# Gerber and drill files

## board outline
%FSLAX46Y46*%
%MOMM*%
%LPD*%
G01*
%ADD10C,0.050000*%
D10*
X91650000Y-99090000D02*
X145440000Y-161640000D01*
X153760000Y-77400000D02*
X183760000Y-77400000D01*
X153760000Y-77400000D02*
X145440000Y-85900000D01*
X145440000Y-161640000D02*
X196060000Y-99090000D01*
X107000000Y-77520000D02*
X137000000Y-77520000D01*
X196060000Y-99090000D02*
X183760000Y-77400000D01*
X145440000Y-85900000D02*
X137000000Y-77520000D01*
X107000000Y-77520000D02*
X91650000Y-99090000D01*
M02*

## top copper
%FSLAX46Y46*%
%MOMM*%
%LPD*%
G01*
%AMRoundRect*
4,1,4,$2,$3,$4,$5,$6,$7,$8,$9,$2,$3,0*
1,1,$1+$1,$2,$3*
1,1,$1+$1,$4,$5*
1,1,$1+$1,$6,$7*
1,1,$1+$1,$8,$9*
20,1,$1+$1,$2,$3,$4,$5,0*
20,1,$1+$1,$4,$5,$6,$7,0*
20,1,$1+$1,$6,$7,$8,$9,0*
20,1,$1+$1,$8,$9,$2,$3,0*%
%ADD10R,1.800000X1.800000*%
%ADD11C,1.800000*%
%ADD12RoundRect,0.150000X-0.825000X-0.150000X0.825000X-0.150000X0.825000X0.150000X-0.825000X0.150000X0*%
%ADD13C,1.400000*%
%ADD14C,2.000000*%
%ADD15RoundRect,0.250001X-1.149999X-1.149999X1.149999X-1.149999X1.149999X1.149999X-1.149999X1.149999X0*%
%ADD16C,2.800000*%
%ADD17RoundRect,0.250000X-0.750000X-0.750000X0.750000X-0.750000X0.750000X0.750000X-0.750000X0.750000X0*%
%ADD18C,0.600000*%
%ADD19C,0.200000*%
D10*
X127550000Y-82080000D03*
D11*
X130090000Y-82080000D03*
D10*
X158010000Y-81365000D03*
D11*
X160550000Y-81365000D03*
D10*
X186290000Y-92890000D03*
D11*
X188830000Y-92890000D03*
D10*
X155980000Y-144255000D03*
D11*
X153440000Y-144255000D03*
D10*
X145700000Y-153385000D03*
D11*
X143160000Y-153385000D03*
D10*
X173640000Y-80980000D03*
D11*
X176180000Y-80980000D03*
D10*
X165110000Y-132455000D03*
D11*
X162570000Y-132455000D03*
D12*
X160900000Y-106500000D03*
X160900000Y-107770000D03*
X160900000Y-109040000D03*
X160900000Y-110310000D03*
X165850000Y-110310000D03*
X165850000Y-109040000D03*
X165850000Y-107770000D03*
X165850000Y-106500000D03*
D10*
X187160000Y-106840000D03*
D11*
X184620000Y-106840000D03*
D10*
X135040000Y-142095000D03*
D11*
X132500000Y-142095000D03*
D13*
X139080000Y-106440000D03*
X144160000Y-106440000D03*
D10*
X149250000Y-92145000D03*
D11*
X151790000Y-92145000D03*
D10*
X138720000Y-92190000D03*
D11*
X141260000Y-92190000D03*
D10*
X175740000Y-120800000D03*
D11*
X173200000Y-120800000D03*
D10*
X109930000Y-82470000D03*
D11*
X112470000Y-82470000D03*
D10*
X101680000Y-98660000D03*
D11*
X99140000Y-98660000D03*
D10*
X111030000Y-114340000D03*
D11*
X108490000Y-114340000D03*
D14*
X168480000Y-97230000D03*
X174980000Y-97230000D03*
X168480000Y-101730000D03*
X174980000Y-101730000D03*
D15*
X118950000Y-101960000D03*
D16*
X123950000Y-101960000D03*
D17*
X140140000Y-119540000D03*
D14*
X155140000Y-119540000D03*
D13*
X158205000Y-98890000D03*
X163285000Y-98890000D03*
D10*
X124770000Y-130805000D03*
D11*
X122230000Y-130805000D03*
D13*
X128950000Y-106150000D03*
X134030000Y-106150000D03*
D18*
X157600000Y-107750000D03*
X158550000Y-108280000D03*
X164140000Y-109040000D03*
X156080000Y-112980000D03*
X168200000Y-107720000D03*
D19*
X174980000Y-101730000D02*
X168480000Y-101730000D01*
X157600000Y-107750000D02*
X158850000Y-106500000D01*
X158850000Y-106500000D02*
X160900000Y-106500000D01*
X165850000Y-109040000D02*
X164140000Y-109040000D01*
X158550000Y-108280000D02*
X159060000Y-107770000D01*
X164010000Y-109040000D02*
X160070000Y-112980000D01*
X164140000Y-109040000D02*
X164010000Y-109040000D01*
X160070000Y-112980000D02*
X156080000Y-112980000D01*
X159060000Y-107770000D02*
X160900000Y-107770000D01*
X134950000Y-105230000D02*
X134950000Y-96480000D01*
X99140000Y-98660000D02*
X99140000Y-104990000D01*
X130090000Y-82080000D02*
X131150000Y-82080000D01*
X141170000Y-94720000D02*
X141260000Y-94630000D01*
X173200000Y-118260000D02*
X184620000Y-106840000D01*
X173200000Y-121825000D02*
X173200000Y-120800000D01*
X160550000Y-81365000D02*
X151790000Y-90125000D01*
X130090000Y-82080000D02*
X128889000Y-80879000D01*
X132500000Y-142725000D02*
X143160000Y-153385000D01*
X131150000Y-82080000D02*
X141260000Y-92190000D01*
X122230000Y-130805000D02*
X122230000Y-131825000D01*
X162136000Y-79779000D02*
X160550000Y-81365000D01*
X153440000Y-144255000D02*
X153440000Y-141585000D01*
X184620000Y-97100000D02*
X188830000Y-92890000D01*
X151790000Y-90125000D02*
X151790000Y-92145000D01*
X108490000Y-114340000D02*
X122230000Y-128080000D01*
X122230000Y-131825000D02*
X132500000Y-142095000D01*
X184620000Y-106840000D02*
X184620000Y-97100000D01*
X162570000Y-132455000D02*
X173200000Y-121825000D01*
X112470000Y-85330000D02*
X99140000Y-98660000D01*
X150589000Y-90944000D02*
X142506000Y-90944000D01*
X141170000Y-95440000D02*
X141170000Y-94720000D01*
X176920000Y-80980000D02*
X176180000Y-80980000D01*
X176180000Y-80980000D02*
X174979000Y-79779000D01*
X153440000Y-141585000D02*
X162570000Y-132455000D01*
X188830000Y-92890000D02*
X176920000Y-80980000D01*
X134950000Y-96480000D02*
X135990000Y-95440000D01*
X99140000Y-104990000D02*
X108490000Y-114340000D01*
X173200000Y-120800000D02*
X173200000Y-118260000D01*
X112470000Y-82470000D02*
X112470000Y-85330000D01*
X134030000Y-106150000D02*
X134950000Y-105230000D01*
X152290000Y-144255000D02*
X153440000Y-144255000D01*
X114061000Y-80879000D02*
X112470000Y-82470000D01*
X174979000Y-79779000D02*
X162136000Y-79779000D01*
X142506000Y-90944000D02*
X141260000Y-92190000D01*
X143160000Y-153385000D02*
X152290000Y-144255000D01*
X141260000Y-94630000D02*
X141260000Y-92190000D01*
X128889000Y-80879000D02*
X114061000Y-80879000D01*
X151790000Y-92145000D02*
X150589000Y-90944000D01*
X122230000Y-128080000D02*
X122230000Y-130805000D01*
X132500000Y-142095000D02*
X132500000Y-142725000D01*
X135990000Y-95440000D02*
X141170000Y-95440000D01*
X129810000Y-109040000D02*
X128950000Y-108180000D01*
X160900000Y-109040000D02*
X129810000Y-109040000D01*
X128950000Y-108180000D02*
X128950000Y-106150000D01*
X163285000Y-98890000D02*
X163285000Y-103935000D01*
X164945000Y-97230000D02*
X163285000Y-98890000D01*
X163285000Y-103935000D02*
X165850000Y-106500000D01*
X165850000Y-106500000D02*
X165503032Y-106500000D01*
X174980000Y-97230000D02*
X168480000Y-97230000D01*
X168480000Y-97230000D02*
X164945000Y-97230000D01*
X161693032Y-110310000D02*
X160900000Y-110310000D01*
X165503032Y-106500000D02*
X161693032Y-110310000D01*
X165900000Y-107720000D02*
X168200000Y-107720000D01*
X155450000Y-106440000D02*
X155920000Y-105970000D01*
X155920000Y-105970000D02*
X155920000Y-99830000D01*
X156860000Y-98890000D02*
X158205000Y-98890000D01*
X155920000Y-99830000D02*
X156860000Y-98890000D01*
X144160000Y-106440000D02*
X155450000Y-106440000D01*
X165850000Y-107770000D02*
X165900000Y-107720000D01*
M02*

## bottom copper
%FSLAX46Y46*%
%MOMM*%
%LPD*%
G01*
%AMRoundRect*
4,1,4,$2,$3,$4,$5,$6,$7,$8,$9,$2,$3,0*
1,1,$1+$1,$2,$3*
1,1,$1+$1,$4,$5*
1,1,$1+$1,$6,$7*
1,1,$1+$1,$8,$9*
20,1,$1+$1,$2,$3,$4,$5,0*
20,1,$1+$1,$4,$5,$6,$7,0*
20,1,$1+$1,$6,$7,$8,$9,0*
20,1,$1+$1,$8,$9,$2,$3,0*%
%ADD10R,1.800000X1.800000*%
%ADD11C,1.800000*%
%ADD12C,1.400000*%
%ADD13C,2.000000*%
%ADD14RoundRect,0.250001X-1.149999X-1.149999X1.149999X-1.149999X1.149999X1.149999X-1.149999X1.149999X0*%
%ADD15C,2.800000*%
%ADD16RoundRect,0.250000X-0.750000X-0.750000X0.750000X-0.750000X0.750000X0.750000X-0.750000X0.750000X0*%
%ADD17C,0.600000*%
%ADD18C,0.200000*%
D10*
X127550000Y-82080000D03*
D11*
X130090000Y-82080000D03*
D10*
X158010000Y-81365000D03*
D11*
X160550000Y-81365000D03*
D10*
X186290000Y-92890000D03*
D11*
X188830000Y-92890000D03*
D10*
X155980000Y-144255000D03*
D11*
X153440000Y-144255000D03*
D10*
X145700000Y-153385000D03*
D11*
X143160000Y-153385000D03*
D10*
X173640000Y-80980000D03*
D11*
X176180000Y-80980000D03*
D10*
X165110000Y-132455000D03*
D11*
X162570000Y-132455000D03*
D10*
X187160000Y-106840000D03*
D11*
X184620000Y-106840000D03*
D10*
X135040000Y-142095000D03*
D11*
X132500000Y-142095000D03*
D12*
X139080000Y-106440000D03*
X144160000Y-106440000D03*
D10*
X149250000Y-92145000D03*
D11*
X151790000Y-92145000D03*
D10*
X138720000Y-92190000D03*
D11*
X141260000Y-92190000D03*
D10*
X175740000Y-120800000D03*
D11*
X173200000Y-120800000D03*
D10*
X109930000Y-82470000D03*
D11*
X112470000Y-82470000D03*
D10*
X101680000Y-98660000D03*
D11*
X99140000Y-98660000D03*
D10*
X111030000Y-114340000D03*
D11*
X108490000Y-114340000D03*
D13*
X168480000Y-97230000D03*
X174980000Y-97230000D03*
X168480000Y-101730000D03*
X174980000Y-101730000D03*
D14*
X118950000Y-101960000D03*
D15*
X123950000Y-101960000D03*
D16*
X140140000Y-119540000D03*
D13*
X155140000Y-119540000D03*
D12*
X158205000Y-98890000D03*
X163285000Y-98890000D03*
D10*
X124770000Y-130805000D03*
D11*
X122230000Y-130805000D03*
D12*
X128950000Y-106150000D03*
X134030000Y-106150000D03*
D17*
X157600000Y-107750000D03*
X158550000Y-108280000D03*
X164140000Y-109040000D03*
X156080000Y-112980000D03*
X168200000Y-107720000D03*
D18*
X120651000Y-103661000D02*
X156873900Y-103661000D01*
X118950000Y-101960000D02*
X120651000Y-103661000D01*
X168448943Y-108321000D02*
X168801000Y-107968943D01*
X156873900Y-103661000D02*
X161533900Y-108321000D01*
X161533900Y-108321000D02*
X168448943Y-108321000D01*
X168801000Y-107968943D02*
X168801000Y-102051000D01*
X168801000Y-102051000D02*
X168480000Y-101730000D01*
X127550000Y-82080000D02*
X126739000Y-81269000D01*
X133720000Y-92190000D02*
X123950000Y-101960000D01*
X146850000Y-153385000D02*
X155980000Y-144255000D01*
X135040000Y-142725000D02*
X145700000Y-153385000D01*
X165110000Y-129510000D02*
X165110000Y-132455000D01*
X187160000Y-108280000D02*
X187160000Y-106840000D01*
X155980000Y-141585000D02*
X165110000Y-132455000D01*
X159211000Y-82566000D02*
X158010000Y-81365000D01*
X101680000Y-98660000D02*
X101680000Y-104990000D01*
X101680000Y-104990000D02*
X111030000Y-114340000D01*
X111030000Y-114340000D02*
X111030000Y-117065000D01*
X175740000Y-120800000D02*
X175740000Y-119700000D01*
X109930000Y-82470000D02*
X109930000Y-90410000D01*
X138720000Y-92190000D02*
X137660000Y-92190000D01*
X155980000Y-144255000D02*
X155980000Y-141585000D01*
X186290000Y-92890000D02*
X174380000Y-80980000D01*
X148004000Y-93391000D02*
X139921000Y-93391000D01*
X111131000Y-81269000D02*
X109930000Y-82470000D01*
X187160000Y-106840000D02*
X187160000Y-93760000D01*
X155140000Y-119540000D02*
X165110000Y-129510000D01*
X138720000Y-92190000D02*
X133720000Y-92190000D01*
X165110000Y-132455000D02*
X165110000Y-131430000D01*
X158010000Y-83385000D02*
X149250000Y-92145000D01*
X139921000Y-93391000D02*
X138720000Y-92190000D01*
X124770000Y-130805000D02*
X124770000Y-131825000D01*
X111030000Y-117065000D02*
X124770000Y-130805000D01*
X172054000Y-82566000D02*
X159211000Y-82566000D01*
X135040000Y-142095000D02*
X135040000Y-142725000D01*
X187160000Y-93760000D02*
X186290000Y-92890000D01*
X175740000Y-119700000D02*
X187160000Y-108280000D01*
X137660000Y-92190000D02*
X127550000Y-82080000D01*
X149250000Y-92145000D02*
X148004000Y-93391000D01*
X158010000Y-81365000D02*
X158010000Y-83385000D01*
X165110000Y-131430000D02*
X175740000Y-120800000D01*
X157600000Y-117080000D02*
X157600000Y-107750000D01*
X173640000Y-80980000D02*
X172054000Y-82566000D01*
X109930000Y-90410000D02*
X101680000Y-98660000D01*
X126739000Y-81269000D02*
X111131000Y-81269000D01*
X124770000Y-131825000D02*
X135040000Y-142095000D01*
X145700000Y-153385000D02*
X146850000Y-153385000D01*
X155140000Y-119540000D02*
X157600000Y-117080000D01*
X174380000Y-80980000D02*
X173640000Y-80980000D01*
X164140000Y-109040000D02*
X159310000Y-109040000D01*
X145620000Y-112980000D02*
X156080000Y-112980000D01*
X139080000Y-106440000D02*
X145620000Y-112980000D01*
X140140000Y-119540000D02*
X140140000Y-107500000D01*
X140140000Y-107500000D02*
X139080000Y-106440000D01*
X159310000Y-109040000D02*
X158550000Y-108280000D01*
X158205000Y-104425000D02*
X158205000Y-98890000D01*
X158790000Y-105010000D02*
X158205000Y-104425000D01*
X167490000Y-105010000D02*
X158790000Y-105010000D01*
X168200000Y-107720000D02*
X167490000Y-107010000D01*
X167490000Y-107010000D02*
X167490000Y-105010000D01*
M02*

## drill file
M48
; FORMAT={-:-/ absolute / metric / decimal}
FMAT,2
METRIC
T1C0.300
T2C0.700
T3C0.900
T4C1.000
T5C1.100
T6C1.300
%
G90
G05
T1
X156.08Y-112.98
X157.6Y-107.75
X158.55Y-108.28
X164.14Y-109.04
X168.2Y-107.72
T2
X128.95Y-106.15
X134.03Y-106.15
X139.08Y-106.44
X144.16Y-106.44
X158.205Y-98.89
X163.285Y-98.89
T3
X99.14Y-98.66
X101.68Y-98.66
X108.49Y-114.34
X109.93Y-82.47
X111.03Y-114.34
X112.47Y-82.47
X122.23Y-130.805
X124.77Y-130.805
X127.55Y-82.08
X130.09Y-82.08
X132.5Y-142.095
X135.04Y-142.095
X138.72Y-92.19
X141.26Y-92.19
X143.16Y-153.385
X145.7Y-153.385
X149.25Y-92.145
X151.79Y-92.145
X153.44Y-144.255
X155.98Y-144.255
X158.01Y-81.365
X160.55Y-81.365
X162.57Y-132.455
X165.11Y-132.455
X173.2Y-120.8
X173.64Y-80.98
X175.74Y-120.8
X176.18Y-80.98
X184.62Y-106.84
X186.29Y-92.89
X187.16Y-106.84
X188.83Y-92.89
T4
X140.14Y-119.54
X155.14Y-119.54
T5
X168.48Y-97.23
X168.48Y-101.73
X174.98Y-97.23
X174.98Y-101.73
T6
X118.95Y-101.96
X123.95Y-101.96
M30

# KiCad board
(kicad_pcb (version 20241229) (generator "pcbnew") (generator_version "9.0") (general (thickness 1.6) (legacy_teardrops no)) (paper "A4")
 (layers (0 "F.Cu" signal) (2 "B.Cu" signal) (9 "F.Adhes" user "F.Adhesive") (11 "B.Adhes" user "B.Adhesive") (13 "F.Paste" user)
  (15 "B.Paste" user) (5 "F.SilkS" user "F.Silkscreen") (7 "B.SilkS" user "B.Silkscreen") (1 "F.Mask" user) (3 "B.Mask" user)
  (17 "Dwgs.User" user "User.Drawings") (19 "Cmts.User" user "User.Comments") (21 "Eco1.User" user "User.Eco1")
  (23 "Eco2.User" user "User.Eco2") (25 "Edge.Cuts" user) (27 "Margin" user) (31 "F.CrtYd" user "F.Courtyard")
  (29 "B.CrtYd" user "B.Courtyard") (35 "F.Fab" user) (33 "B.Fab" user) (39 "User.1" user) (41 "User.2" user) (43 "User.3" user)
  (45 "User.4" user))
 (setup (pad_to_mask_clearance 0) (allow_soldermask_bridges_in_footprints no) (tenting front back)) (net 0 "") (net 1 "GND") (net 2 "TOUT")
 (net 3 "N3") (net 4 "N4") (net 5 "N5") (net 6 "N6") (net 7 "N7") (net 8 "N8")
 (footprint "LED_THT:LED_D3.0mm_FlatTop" (layer "F.Cu") (at 127.55 82.08)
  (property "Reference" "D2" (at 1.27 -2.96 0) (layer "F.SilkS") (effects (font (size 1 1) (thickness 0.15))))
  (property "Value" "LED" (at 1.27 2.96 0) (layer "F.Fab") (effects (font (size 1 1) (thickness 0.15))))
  (pad "1" thru_hole rect (at 0 0) (size 1.8 1.8) (drill 0.9) (layers "*.Cu" "*.Mask") (remove_unused_layers no) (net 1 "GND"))
  (pad "2" thru_hole circle (at 2.54 0) (size 1.8 1.8) (drill 0.9) (layers "*.Cu" "*.Mask") (remove_unused_layers no) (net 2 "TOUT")))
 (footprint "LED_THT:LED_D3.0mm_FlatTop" (layer "F.Cu") (at 158.01 81.365)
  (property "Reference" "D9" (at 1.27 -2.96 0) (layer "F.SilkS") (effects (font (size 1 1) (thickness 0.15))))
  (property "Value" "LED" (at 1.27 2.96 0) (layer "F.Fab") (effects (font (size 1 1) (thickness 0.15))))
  (pad "1" thru_hole rect (at 0 0) (size 1.8 1.8) (drill 0.9) (layers "*.Cu" "*.Mask") (remove_unused_layers no) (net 1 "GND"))
  (pad "2" thru_hole circle (at 2.54 0) (size 1.8 1.8) (drill 0.9) (layers "*.Cu" "*.Mask") (remove_unused_layers no) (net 2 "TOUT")))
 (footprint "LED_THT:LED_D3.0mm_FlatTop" (layer "F.Cu") (at 186.29 92.89)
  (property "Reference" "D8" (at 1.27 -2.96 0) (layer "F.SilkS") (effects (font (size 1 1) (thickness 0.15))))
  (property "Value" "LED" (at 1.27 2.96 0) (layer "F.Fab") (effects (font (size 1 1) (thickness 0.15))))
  (pad "1" thru_hole rect (at 0 0) (size 1.8 1.8) (drill 0.9) (layers "*.Cu" "*.Mask") (remove_unused_layers no) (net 1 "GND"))
  (pad "2" thru_hole circle (at 2.54 0) (size 1.8 1.8) (drill 0.9) (layers "*.Cu" "*.Mask") (remove_unused_layers no) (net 2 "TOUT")))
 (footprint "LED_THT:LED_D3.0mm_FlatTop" (layer "F.Cu") (at 155.98 144.255 180)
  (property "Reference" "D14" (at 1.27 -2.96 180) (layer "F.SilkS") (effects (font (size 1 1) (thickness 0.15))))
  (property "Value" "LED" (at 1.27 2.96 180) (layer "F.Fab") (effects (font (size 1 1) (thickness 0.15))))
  (pad "1" thru_hole rect (at 0 0 180) (size 1.8 1.8) (drill 0.9) (layers "*.Cu" "*.Mask") (remove_unused_layers no) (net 1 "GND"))
  (pad "2" thru_hole circle (at 2.54 0 180) (size 1.8 1.8) (drill 0.9) (layers "*.Cu" "*.Mask") (remove_unused_layers no) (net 2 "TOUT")))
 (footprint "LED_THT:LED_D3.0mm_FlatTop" (layer "F.Cu") (at 145.7 153.385 180)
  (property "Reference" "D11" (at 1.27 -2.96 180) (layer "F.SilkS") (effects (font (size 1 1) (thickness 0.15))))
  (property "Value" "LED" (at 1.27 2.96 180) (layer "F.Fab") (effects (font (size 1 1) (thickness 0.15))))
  (pad "1" thru_hole rect (at 0 0 180) (size 1.8 1.8) (drill 0.9) (layers "*.Cu" "*.Mask") (remove_unused_layers no) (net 1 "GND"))
  (pad "2" thru_hole circle (at 2.54 0 180) (size 1.8 1.8) (drill 0.9) (layers "*.Cu" "*.Mask") (remove_unused_layers no) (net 2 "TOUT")))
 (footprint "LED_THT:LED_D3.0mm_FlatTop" (layer "F.Cu") (at 173.64 80.98)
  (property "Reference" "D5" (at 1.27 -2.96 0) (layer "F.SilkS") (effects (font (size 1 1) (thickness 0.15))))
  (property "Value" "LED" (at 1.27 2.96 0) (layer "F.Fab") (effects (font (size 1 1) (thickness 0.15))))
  (pad "1" thru_hole rect (at 0 0) (size 1.8 1.8) (drill 0.9) (layers "*.Cu" "*.Mask") (remove_unused_layers no) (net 1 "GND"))
  (pad "2" thru_hole circle (at 2.54 0) (size 1.8 1.8) (drill 0.9) (layers "*.Cu" "*.Mask") (remove_unused_layers no) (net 2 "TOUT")))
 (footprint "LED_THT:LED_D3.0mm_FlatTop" (layer "F.Cu") (at 165.11 132.455 180)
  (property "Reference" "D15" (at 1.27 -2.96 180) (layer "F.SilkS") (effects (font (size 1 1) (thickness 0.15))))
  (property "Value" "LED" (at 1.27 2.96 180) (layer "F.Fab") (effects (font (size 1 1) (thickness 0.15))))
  (pad "1" thru_hole rect (at 0 0 180) (size 1.8 1.8) (drill 0.9) (layers "*.Cu" "*.Mask") (remove_unused_layers no) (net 1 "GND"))
  (pad "2" thru_hole circle (at 2.54 0 180) (size 1.8 1.8) (drill 0.9) (layers "*.Cu" "*.Mask") (remove_unused_layers no) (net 2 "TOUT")))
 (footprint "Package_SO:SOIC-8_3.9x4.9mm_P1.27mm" (layer "F.Cu") (at 163.375 108.405)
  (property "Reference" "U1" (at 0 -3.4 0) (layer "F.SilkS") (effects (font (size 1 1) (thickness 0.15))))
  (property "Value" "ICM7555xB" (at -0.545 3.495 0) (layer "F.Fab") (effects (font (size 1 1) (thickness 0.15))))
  (pad "1" smd roundrect (at -2.475 -1.905) (size 1.95 0.6) (layers "F.Cu" "F.Mask" "F.Paste") (roundrect_rratio 0.25) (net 1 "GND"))
  (pad "2" smd roundrect (at -2.475 -0.635) (size 1.95 0.6) (layers "F.Cu" "F.Mask" "F.Paste") (roundrect_rratio 0.25) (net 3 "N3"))
  (pad "3" smd roundrect (at -2.475 0.635) (size 1.95 0.6) (layers "F.Cu" "F.Mask" "F.Paste") (roundrect_rratio 0.25) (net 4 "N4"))
  (pad "4" smd roundrect (at -2.475 1.905) (size 1.95 0.6) (layers "F.Cu" "F.Mask" "F.Paste") (roundrect_rratio 0.25) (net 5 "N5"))
  (pad "5" smd roundrect (at 2.475 1.905) (size 1.95 0.6) (layers "F.Cu" "F.Mask" "F.Paste") (roundrect_rratio 0.25) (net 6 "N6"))
  (pad "6" smd roundrect (at 2.475 0.635) (size 1.95 0.6) (layers "F.Cu" "F.Mask" "F.Paste") (roundrect_rratio 0.25) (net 3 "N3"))
  (pad "7" smd roundrect (at 2.475 -0.635) (size 1.95 0.6) (layers "F.Cu" "F.Mask" "F.Paste") (roundrect_rratio 0.25) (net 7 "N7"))
  (pad "8" smd roundrect (at 2.475 -1.905) (size 1.95 0.6) (layers "F.Cu" "F.Mask" "F.Paste") (roundrect_rratio 0.25) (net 5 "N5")))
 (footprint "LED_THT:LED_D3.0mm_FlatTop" (layer "F.Cu") (at 187.16 106.84 180)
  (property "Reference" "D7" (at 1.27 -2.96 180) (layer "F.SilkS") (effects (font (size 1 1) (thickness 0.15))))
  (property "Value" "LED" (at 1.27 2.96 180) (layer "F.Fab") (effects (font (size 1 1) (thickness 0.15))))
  (pad "1" thru_hole rect (at 0 0 180) (size 1.8 1.8) (drill 0.9) (layers "*.Cu" "*.Mask") (remove_unused_layers no) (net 1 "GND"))
  (pad "2" thru_hole circle (at 2.54 0 180) (size 1.8 1.8) (drill 0.9) (layers "*.Cu" "*.Mask") (remove_unused_layers no) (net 2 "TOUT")))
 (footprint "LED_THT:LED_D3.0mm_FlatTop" (layer "F.Cu") (at 135.04 142.095 180)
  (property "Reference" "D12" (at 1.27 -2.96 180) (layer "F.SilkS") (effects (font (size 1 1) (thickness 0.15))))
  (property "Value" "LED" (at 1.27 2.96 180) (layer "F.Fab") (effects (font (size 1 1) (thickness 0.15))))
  (pad "1" thru_hole rect (at 0 0 180) (size 1.8 1.8) (drill 0.9) (layers "*.Cu" "*.Mask") (remove_unused_layers no) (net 1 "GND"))
  (pad "2" thru_hole circle (at 2.54 0 180) (size 1.8 1.8) (drill 0.9) (layers "*.Cu" "*.Mask") (remove_unused_layers no) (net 2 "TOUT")))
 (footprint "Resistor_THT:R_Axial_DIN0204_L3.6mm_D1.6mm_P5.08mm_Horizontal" (layer "F.Cu") (at 139.08 106.44)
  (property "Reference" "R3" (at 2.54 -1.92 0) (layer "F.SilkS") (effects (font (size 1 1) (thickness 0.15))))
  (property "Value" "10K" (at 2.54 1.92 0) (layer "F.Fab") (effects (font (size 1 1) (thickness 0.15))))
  (pad "1" thru_hole circle (at 0 0) (size 1.4 1.4) (drill 0.7) (layers "*.Cu" "*.Mask") (remove_unused_layers no) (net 3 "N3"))
  (pad "2" thru_hole circle (at 5.08 0) (size 1.4 1.4) (drill 0.7) (layers "*.Cu" "*.Mask") (remove_unused_layers no) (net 7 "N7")))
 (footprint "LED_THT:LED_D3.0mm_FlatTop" (layer "F.Cu") (at 149.25 92.145)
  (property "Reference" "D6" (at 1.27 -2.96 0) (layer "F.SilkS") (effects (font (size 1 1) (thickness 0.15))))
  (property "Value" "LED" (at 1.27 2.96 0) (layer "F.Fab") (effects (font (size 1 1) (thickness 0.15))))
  (pad "1" thru_hole rect (at 0 0) (size 1.8 1.8) (drill 0.9) (layers "*.Cu" "*.Mask") (remove_unused_layers no) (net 1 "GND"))
  (pad "2" thru_hole circle (at 2.54 0) (size 1.8 1.8) (drill 0.9) (layers "*.Cu" "*.Mask") (remove_unused_layers no) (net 2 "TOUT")))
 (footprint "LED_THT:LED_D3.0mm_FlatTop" (layer "F.Cu") (at 138.72 92.19)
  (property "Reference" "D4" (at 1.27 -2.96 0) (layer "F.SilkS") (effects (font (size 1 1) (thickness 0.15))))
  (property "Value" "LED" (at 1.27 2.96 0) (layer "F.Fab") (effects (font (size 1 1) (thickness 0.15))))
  (pad "1" thru_hole rect (at 0 0) (size 1.8 1.8) (drill 0.9) (layers "*.Cu" "*.Mask") (remove_unused_layers no) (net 1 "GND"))
  (pad "2" thru_hole circle (at 2.54 0) (size 1.8 1.8) (drill 0.9) (layers "*.Cu" "*.Mask") (remove_unused_layers no) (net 2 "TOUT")))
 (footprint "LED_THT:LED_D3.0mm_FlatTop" (layer "F.Cu") (at 175.74 120.8 180)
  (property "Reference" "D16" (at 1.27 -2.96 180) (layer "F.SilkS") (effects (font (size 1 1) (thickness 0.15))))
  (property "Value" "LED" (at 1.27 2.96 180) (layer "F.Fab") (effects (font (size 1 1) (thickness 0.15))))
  (pad "1" thru_hole rect (at 0 0 180) (size 1.8 1.8) (drill 0.9) (layers "*.Cu" "*.Mask") (remove_unused_layers no) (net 1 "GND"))
  (pad "2" thru_hole circle (at 2.54 0 180) (size 1.8 1.8) (drill 0.9) (layers "*.Cu" "*.Mask") (remove_unused_layers no) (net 2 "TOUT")))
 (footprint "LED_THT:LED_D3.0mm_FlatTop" (layer "F.Cu") (at 109.93 82.47)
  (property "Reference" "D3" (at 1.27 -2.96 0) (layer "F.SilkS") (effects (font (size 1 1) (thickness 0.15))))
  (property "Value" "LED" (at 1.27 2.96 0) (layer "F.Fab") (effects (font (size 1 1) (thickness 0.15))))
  (pad "1" thru_hole rect (at 0 0) (size 1.8 1.8) (drill 0.9) (layers "*.Cu" "*.Mask") (remove_unused_layers no) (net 1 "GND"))
  (pad "2" thru_hole circle (at 2.54 0) (size 1.8 1.8) (drill 0.9) (layers "*.Cu" "*.Mask") (remove_unused_layers no) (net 2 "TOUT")))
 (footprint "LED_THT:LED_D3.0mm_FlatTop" (layer "F.Cu") (at 101.68 98.66 180)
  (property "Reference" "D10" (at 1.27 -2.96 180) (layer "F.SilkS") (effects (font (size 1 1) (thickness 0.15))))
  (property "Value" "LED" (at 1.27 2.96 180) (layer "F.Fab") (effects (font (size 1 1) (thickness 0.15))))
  (pad "1" thru_hole rect (at 0 0 180) (size 1.8 1.8) (drill 0.9) (layers "*.Cu" "*.Mask") (remove_unused_layers no) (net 1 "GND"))
  (pad "2" thru_hole circle (at 2.54 0 180) (size 1.8 1.8) (drill 0.9) (layers "*.Cu" "*.Mask") (remove_unused_layers no) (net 2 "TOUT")))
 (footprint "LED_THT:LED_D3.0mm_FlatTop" (layer "F.Cu") (at 111.03 114.34 180)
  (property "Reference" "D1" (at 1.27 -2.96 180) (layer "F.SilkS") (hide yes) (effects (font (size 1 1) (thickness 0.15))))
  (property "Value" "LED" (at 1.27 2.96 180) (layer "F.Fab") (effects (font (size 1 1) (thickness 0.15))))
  (pad "1" thru_hole rect (at 0 0 180) (size 1.8 1.8) (drill 0.9) (layers "*.Cu" "*.Mask") (remove_unused_layers no) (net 1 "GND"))
  (pad "2" thru_hole circle (at 2.54 0 180) (size 1.8 1.8) (drill 0.9) (layers "*.Cu" "*.Mask") (remove_unused_layers no) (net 2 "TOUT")))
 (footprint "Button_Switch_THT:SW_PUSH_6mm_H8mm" (layer "F.Cu") (at 168.48 97.23)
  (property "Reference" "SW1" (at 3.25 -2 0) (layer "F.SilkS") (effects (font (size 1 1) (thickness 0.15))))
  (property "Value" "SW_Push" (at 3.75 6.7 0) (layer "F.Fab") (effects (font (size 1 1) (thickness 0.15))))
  (pad "1" thru_hole circle (at 0 0 90) (size 2 2) (drill 1.1) (layers "*.Cu" "*.Mask") (remove_unused_layers no) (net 5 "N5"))
  (pad "1" thru_hole circle (at 6.5 0 90) (size 2 2) (drill 1.1) (layers "*.Cu" "*.Mask") (remove_unused_layers no) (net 5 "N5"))
  (pad "2" thru_hole circle (at 0 4.5 90) (size 2 2) (drill 1.1) (layers "*.Cu" "*.Mask") (remove_unused_layers no) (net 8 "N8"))
  (pad "2" thru_hole circle (at 6.5 4.5 90) (size 2 2) (drill 1.1) (layers "*.Cu" "*.Mask") (remove_unused_layers no) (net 8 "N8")))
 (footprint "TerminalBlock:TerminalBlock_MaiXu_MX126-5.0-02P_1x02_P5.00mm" (layer "F.Cu") (at 118.95 101.96)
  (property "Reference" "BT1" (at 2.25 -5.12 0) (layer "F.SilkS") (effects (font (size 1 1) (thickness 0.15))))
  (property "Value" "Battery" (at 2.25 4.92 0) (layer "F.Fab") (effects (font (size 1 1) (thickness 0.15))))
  (pad "1" thru_hole roundrect (at 0 0) (size 2.8 2.8) (drill 1.3) (layers "*.Cu" "*.Mask") (remove_unused_layers no)
   (roundrect_rratio 0.089286) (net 8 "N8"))
  (pad "2" thru_hole circle (at 5 0) (size 2.8 2.8) (drill 1.3) (layers "*.Cu" "*.Mask") (remove_unused_layers no) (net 1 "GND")))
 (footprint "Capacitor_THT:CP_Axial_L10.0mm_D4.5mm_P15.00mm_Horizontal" (layer "F.Cu") (at 140.14 119.54)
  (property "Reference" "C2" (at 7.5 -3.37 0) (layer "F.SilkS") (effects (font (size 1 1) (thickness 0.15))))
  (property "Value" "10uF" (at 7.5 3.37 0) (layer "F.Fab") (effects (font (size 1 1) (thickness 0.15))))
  (pad "1" thru_hole roundrect (at 0 0) (size 2 2) (drill 1) (layers "*.Cu" "*.Mask") (remove_unused_layers no) (roundrect_rratio 0.125)
   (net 3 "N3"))
  (pad "2" thru_hole circle (at 15 0) (size 2 2) (drill 1) (layers "*.Cu" "*.Mask") (remove_unused_layers no) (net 1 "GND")))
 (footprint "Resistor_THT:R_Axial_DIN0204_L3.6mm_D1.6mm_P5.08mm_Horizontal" (layer "F.Cu") (at 158.205 98.89)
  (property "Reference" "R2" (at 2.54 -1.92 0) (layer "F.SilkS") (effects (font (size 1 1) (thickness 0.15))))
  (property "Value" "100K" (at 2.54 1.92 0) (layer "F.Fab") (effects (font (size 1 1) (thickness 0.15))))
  (pad "1" thru_hole circle (at 0 0) (size 1.4 1.4) (drill 0.7) (layers "*.Cu" "*.Mask") (remove_unused_layers no) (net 7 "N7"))
  (pad "2" thru_hole circle (at 5.08 0) (size 1.4 1.4) (drill 0.7) (layers "*.Cu" "*.Mask") (remove_unused_layers no) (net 5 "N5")))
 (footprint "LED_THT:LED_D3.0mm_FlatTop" (layer "F.Cu") (at 124.77 130.805 180)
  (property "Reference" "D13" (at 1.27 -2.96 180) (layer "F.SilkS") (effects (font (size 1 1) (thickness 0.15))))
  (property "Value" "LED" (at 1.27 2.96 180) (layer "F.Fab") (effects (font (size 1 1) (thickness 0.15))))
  (pad "1" thru_hole rect (at 0 0 180) (size 1.8 1.8) (drill 0.9) (layers "*.Cu" "*.Mask") (remove_unused_layers no) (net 1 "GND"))
  (pad "2" thru_hole circle (at 2.54 0 180) (size 1.8 1.8) (drill 0.9) (layers "*.Cu" "*.Mask") (remove_unused_layers no) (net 2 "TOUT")))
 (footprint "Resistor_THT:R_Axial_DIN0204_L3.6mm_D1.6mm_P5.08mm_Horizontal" (layer "F.Cu") (at 128.95 106.15)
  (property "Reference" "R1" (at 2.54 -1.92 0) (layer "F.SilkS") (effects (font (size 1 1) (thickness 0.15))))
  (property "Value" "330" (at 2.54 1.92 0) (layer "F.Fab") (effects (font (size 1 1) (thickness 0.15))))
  (pad "1" thru_hole circle (at 0 0) (size 1.4 1.4) (drill 0.7) (layers "*.Cu" "*.Mask") (remove_unused_layers no) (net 4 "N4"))
  (pad "2" thru_hole circle (at 5.08 0) (size 1.4 1.4) (drill 0.7) (layers "*.Cu" "*.Mask") (remove_unused_layers no) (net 2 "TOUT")))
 (gr_line (start 91.65 99.09) (end 145.44 161.64) (stroke (width 0.05) (type default)) (layer "Edge.Cuts"))
 (gr_line (start 153.76 77.4) (end 183.76 77.4) (stroke (width 0.05) (type solid)) (layer "Edge.Cuts"))
 (gr_line (start 153.76 77.4) (end 145.44 85.9) (stroke (width 0.05) (type default)) (layer "Edge.Cuts"))
 (gr_line (start 145.44 161.64) (end 196.06 99.09) (stroke (width 0.05) (type default)) (layer "Edge.Cuts"))
 (gr_line (start 107 77.52) (end 137 77.52) (stroke (width 0.05) (type solid)) (layer "Edge.Cuts"))
 (gr_line (start 196.06 99.09) (end 183.76 77.4) (stroke (width 0.05) (type default)) (layer "Edge.Cuts"))
 (gr_line (start 145.44 85.9) (end 137 77.52) (stroke (width 0.05) (type default)) (layer "Edge.Cuts"))
 (gr_line (start 107 77.52) (end 91.65 99.09) (stroke (width 0.05) (type default)) (layer "Edge.Cuts"))
 (segment (start 174.98 101.73) (end 168.48 101.73) (width 0.2) (layer "F.Cu") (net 8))
 (segment (start 120.651 103.661) (end 156.8739 103.661) (width 0.2) (layer "B.Cu") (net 8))
 (segment (start 118.95 101.96) (end 120.651 103.661) (width 0.2) (layer "B.Cu") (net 8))
 (segment (start 168.448943 108.321) (end 168.801 107.968943) (width 0.2) (layer "B.Cu") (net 8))
 (segment (start 156.8739 103.661) (end 161.5339 108.321) (width 0.2) (layer "B.Cu") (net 8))
 (segment (start 161.5339 108.321) (end 168.448943 108.321) (width 0.2) (layer "B.Cu") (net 8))
 (segment (start 168.801 107.968943) (end 168.801 102.051) (width 0.2) (layer "B.Cu") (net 8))
 (segment (start 168.801 102.051) (end 168.48 101.73) (width 0.2) (layer "B.Cu") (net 8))
 (segment (start 157.6 107.75) (end 158.85 106.5) (width 0.2) (layer "F.Cu") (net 1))
 (segment (start 158.85 106.5) (end 160.9 106.5) (width 0.2) (layer "F.Cu") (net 1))
 (via (at 157.6 107.75) (size 0.6) (drill 0.3) (layers "F.Cu" "B.Cu") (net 1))
 (segment (start 127.55 82.08) (end 126.739 81.269) (width 0.2) (layer "B.Cu") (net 1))
 (segment (start 133.72 92.19) (end 123.95 101.96) (width 0.2) (layer "B.Cu") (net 1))
 (segment (start 146.85 153.385) (end 155.98 144.255) (width 0.2) (layer "B.Cu") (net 1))
 (segment (start 135.04 142.725) (end 145.7 153.385) (width 0.2) (layer "B.Cu") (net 1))
 (segment (start 165.11 129.51) (end 165.11 132.455) (width 0.2) (layer "B.Cu") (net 1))
 (segment (start 187.16 108.28) (end 187.16 106.84) (width 0.2) (layer "B.Cu") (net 1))
 (segment (start 155.98 141.585) (end 165.11 132.455) (width 0.2) (layer "B.Cu") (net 1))
 (segment (start 159.211 82.566) (end 158.01 81.365) (width 0.2) (layer "B.Cu") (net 1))
 (segment (start 101.68 98.66) (end 101.68 104.99) (width 0.2) (layer "B.Cu") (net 1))
 (segment (start 101.68 104.99) (end 111.03 114.34) (width 0.2) (layer "B.Cu") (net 1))
 (segment (start 111.03 114.34) (end 111.03 117.065) (width 0.2) (layer "B.Cu") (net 1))
 (segment (start 175.74 120.8) (end 175.74 119.7) (width 0.2) (layer "B.Cu") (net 1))
 (segment (start 109.93 82.47) (end 109.93 90.41) (width 0.2) (layer "B.Cu") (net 1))
 (segment (start 138.72 92.19) (end 137.66 92.19) (width 0.2) (layer "B.Cu") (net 1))
 (segment (start 155.98 144.255) (end 155.98 141.585) (width 0.2) (layer "B.Cu") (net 1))
 (segment (start 186.29 92.89) (end 174.38 80.98) (width 0.2) (layer "B.Cu") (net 1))
 (segment (start 148.004 93.391) (end 139.921 93.391) (width 0.2) (layer "B.Cu") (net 1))
 (segment (start 111.131 81.269) (end 109.93 82.47) (width 0.2) (layer "B.Cu") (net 1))
 (segment (start 187.16 106.84) (end 187.16 93.76) (width 0.2) (layer "B.Cu") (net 1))
 (segment (start 155.14 119.54) (end 165.11 129.51) (width 0.2) (layer "B.Cu") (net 1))
 (segment (start 138.72 92.19) (end 133.72 92.19) (width 0.2) (layer "B.Cu") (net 1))
 (segment (start 165.11 132.455) (end 165.11 131.43) (width 0.2) (layer "B.Cu") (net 1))
 (segment (start 158.01 83.385) (end 149.25 92.145) (width 0.2) (layer "B.Cu") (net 1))
 (segment (start 139.921 93.391) (end 138.72 92.19) (width 0.2) (layer "B.Cu") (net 1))
 (segment (start 124.77 130.805) (end 124.77 131.825) (width 0.2) (layer "B.Cu") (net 1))
 (segment (start 111.03 117.065) (end 124.77 130.805) (width 0.2) (layer "B.Cu") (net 1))
 (segment (start 172.054 82.566) (end 159.211 82.566) (width 0.2) (layer "B.Cu") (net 1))
 (segment (start 135.04 142.095) (end 135.04 142.725) (width 0.2) (layer "B.Cu") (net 1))
 (segment (start 187.16 93.76) (end 186.29 92.89) (width 0.2) (layer "B.Cu") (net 1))
 (segment (start 175.74 119.7) (end 187.16 108.28) (width 0.2) (layer "B.Cu") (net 1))
 (segment (start 137.66 92.19) (end 127.55 82.08) (width 0.2) (layer "B.Cu") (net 1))
 (segment (start 149.25 92.145) (end 148.004 93.391) (width 0.2) (layer "B.Cu") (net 1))
 (segment (start 158.01 81.365) (end 158.01 83.385) (width 0.2) (layer "B.Cu") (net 1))
 (segment (start 165.11 131.43) (end 175.74 120.8) (width 0.2) (layer "B.Cu") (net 1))
 (segment (start 157.6 117.08) (end 157.6 107.75) (width 0.2) (layer "B.Cu") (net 1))
 (segment (start 173.64 80.98) (end 172.054 82.566) (width 0.2) (layer "B.Cu") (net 1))
 (segment (start 109.93 90.41) (end 101.68 98.66) (width 0.2) (layer "B.Cu") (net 1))
 (segment (start 126.739 81.269) (end 111.131 81.269) (width 0.2) (layer "B.Cu") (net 1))
 (segment (start 124.77 131.825) (end 135.04 142.095) (width 0.2) (layer "B.Cu") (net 1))
 (segment (start 145.7 153.385) (end 146.85 153.385) (width 0.2) (layer "B.Cu") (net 1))
 (segment (start 155.14 119.54) (end 157.6 117.08) (width 0.2) (layer "B.Cu") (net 1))
 (segment (start 174.38 80.98) (end 173.64 80.98) (width 0.2) (layer "B.Cu") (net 1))
 (segment (start 165.85 109.04) (end 164.14 109.04) (width 0.2) (layer "F.Cu") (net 3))
 (segment (start 158.55 108.28) (end 159.06 107.77) (width 0.2) (layer "F.Cu") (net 3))
 (segment (start 164.01 109.04) (end 160.07 112.98) (width 0.2) (layer "F.Cu") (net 3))
 (segment (start 164.14 109.04) (end 164.01 109.04) (width 0.2) (layer "F.Cu") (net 3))
 (segment (start 160.07 112.98) (end 156.08 112.98) (width 0.2) (layer "F.Cu") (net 3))
 (segment (start 159.06 107.77) (end 160.9 107.77) (width 0.2) (layer "F.Cu") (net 3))
 (via (at 158.55 108.28) (size 0.6) (drill 0.3) (layers "F.Cu" "B.Cu") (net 3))
 (via (at 164.14 109.04) (size 0.6) (drill 0.3) (layers "F.Cu" "B.Cu") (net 3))
 (via (at 156.08 112.98) (size 0.6) (drill 0.3) (layers "F.Cu" "B.Cu") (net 3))
 (segment (start 164.14 109.04) (end 159.31 109.04) (width 0.2) (layer "B.Cu") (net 3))
 (segment (start 145.62 112.98) (end 156.08 112.98) (width 0.2) (layer "B.Cu") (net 3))
 (segment (start 139.08 106.44) (end 145.62 112.98) (width 0.2) (layer "B.Cu") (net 3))
 (segment (start 140.14 119.54) (end 140.14 107.5) (width 0.2) (layer "B.Cu") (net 3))
 (segment (start 140.14 107.5) (end 139.08 106.44) (width 0.2) (layer "B.Cu") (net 3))
 (segment (start 159.31 109.04) (end 158.55 108.28) (width 0.2) (layer "B.Cu") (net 3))
 (segment (start 134.95 105.23) (end 134.95 96.48) (width 0.2) (layer "F.Cu") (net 2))
 (segment (start 99.14 98.66) (end 99.14 104.99) (width 0.2) (layer "F.Cu") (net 2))
 (segment (start 130.09 82.08) (end 131.15 82.08) (width 0.2) (layer "F.Cu") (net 2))
 (segment (start 141.17 94.72) (end 141.26 94.63) (width 0.2) (layer "F.Cu") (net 2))
 (segment (start 173.2 118.26) (end 184.62 106.84) (width 0.2) (layer "F.Cu") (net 2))
 (segment (start 173.2 121.825) (end 173.2 120.8) (width 0.2) (layer "F.Cu") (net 2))
 (segment (start 160.55 81.365) (end 151.79 90.125) (width 0.2) (layer "F.Cu") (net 2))
 (segment (start 130.09 82.08) (end 128.889 80.879) (width 0.2) (layer "F.Cu") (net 2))
 (segment (start 132.5 142.725) (end 143.16 153.385) (width 0.2) (layer "F.Cu") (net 2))
 (segment (start 131.15 82.08) (end 141.26 92.19) (width 0.2) (layer "F.Cu") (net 2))
 (segment (start 122.23 130.805) (end 122.23 131.825) (width 0.2) (layer "F.Cu") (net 2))
 (segment (start 162.136 79.779) (end 160.55 81.365) (width 0.2) (layer "F.Cu") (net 2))
 (segment (start 153.44 144.255) (end 153.44 141.585) (width 0.2) (layer "F.Cu") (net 2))
 (segment (start 184.62 97.1) (end 188.83 92.89) (width 0.2) (layer "F.Cu") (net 2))
 (segment (start 151.79 90.125) (end 151.79 92.145) (width 0.2) (layer "F.Cu") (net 2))
 (segment (start 108.49 114.34) (end 122.23 128.08) (width 0.2) (layer "F.Cu") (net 2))
 (segment (start 122.23 131.825) (end 132.5 142.095) (width 0.2) (layer "F.Cu") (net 2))
 (segment (start 184.62 106.84) (end 184.62 97.1) (width 0.2) (layer "F.Cu") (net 2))
 (segment (start 162.57 132.455) (end 173.2 121.825) (width 0.2) (layer "F.Cu") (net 2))
 (segment (start 112.47 85.33) (end 99.14 98.66) (width 0.2) (layer "F.Cu") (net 2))
 (segment (start 150.589 90.944) (end 142.506 90.944) (width 0.2) (layer "F.Cu") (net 2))
 (segment (start 141.17 95.44) (end 141.17 94.72) (width 0.2) (layer "F.Cu") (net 2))
 (segment (start 176.92 80.98) (end 176.18 80.98) (width 0.2) (layer "F.Cu") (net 2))
 (segment (start 176.18 80.98) (end 174.979 79.779) (width 0.2) (layer "F.Cu") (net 2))
 (segment (start 153.44 141.585) (end 162.57 132.455) (width 0.2) (layer "F.Cu") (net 2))
 (segment (start 188.83 92.89) (end 176.92 80.98) (width 0.2) (layer "F.Cu") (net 2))
 (segment (start 134.95 96.48) (end 135.99 95.44) (width 0.2) (layer "F.Cu") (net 2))
 (segment (start 99.14 104.99) (end 108.49 114.34) (width 0.2) (layer "F.Cu") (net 2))
 (segment (start 173.2 120.8) (end 173.2 118.26) (width 0.2) (layer "F.Cu") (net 2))
 (segment (start 112.47 82.47) (end 112.47 85.33) (width 0.2) (layer "F.Cu") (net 2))
 (segment (start 134.03 106.15) (end 134.95 105.23) (width 0.2) (layer "F.Cu") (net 2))
 (segment (start 152.29 144.255) (end 153.44 144.255) (width 0.2) (layer "F.Cu") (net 2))
 (segment (start 114.061 80.879) (end 112.47 82.47) (width 0.2) (layer "F.Cu") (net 2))
 (segment (start 174.979 79.779) (end 162.136 79.779) (width 0.2) (layer "F.Cu") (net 2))
 (segment (start 142.506 90.944) (end 141.26 92.19) (width 0.2) (layer "F.Cu") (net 2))
 (segment (start 143.16 153.385) (end 152.29 144.255) (width 0.2) (layer "F.Cu") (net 2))
 (segment (start 141.26 94.63) (end 141.26 92.19) (width 0.2) (layer "F.Cu") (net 2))
 (segment (start 128.889 80.879) (end 114.061 80.879) (width 0.2) (layer "F.Cu") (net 2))
 (segment (start 151.79 92.145) (end 150.589 90.944) (width 0.2) (layer "F.Cu") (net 2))
 (segment (start 122.23 128.08) (end 122.23 130.805) (width 0.2) (layer "F.Cu") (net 2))
 (segment (start 132.5 142.095) (end 132.5 142.725) (width 0.2) (layer "F.Cu") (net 2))
 (segment (start 135.99 95.44) (end 141.17 95.44) (width 0.2) (layer "F.Cu") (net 2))
 (segment (start 129.81 109.04) (end 128.95 108.18) (width 0.2) (layer "F.Cu") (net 4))
 (segment (start 160.9 109.04) (end 129.81 109.04) (width 0.2) (layer "F.Cu") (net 4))
 (segment (start 128.95 108.18) (end 128.95 106.15) (width 0.2) (layer "F.Cu") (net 4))
 (segment (start 163.285 98.89) (end 163.285 103.935) (width 0.2) (layer "F.Cu") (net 5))
 (segment (start 164.945 97.23) (end 163.285 98.89) (width 0.2) (layer "F.Cu") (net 5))
 (segment (start 163.285 103.935) (end 165.85 106.5) (width 0.2) (layer "F.Cu") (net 5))
 (segment (start 165.85 106.5) (end 165.503032 106.5) (width 0.2) (layer "F.Cu") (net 5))
 (segment (start 174.98 97.23) (end 168.48 97.23) (width 0.2) (layer "F.Cu") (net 5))
 (segment (start 168.48 97.23) (end 164.945 97.23) (width 0.2) (layer "F.Cu") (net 5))
 (segment (start 161.693032 110.31) (end 160.9 110.31) (width 0.2) (layer "F.Cu") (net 5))
 (segment (start 165.503032 106.5) (end 161.693032 110.31) (width 0.2) (layer "F.Cu") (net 5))
 (segment (start 165.9 107.72) (end 168.2 107.72) (width 0.2) (layer "F.Cu") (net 7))
 (segment (start 155.45 106.44) (end 155.92 105.97) (width 0.2) (layer "F.Cu") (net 7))
 (segment (start 155.92 105.97) (end 155.92 99.83) (width 0.2) (layer "F.Cu") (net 7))
 (segment (start 156.86 98.89) (end 158.205 98.89) (width 0.2) (layer "F.Cu") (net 7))
 (segment (start 155.92 99.83) (end 156.86 98.89) (width 0.2) (layer "F.Cu") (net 7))
 (segment (start 144.16 106.44) (end 155.45 106.44) (width 0.2) (layer "F.Cu") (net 7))
 (segment (start 165.85 107.77) (end 165.9 107.72) (width 0.2) (layer "F.Cu") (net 7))
 (via (at 168.2 107.72) (size 0.6) (drill 0.3) (layers "F.Cu" "B.Cu") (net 7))
 (segment (start 158.205 104.425) (end 158.205 98.89) (width 0.2) (layer "B.Cu") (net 7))
 (segment (start 158.79 105.01) (end 158.205 104.425) (width 0.2) (layer "B.Cu") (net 7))
 (segment (start 167.49 105.01) (end 158.79 105.01) (width 0.2) (layer "B.Cu") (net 7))
 (segment (start 168.2 107.72) (end 167.49 107.01) (width 0.2) (layer "B.Cu") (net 7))
 (segment (start 167.49 107.01) (end 167.49 105.01) (width 0.2) (layer "B.Cu") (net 7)))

